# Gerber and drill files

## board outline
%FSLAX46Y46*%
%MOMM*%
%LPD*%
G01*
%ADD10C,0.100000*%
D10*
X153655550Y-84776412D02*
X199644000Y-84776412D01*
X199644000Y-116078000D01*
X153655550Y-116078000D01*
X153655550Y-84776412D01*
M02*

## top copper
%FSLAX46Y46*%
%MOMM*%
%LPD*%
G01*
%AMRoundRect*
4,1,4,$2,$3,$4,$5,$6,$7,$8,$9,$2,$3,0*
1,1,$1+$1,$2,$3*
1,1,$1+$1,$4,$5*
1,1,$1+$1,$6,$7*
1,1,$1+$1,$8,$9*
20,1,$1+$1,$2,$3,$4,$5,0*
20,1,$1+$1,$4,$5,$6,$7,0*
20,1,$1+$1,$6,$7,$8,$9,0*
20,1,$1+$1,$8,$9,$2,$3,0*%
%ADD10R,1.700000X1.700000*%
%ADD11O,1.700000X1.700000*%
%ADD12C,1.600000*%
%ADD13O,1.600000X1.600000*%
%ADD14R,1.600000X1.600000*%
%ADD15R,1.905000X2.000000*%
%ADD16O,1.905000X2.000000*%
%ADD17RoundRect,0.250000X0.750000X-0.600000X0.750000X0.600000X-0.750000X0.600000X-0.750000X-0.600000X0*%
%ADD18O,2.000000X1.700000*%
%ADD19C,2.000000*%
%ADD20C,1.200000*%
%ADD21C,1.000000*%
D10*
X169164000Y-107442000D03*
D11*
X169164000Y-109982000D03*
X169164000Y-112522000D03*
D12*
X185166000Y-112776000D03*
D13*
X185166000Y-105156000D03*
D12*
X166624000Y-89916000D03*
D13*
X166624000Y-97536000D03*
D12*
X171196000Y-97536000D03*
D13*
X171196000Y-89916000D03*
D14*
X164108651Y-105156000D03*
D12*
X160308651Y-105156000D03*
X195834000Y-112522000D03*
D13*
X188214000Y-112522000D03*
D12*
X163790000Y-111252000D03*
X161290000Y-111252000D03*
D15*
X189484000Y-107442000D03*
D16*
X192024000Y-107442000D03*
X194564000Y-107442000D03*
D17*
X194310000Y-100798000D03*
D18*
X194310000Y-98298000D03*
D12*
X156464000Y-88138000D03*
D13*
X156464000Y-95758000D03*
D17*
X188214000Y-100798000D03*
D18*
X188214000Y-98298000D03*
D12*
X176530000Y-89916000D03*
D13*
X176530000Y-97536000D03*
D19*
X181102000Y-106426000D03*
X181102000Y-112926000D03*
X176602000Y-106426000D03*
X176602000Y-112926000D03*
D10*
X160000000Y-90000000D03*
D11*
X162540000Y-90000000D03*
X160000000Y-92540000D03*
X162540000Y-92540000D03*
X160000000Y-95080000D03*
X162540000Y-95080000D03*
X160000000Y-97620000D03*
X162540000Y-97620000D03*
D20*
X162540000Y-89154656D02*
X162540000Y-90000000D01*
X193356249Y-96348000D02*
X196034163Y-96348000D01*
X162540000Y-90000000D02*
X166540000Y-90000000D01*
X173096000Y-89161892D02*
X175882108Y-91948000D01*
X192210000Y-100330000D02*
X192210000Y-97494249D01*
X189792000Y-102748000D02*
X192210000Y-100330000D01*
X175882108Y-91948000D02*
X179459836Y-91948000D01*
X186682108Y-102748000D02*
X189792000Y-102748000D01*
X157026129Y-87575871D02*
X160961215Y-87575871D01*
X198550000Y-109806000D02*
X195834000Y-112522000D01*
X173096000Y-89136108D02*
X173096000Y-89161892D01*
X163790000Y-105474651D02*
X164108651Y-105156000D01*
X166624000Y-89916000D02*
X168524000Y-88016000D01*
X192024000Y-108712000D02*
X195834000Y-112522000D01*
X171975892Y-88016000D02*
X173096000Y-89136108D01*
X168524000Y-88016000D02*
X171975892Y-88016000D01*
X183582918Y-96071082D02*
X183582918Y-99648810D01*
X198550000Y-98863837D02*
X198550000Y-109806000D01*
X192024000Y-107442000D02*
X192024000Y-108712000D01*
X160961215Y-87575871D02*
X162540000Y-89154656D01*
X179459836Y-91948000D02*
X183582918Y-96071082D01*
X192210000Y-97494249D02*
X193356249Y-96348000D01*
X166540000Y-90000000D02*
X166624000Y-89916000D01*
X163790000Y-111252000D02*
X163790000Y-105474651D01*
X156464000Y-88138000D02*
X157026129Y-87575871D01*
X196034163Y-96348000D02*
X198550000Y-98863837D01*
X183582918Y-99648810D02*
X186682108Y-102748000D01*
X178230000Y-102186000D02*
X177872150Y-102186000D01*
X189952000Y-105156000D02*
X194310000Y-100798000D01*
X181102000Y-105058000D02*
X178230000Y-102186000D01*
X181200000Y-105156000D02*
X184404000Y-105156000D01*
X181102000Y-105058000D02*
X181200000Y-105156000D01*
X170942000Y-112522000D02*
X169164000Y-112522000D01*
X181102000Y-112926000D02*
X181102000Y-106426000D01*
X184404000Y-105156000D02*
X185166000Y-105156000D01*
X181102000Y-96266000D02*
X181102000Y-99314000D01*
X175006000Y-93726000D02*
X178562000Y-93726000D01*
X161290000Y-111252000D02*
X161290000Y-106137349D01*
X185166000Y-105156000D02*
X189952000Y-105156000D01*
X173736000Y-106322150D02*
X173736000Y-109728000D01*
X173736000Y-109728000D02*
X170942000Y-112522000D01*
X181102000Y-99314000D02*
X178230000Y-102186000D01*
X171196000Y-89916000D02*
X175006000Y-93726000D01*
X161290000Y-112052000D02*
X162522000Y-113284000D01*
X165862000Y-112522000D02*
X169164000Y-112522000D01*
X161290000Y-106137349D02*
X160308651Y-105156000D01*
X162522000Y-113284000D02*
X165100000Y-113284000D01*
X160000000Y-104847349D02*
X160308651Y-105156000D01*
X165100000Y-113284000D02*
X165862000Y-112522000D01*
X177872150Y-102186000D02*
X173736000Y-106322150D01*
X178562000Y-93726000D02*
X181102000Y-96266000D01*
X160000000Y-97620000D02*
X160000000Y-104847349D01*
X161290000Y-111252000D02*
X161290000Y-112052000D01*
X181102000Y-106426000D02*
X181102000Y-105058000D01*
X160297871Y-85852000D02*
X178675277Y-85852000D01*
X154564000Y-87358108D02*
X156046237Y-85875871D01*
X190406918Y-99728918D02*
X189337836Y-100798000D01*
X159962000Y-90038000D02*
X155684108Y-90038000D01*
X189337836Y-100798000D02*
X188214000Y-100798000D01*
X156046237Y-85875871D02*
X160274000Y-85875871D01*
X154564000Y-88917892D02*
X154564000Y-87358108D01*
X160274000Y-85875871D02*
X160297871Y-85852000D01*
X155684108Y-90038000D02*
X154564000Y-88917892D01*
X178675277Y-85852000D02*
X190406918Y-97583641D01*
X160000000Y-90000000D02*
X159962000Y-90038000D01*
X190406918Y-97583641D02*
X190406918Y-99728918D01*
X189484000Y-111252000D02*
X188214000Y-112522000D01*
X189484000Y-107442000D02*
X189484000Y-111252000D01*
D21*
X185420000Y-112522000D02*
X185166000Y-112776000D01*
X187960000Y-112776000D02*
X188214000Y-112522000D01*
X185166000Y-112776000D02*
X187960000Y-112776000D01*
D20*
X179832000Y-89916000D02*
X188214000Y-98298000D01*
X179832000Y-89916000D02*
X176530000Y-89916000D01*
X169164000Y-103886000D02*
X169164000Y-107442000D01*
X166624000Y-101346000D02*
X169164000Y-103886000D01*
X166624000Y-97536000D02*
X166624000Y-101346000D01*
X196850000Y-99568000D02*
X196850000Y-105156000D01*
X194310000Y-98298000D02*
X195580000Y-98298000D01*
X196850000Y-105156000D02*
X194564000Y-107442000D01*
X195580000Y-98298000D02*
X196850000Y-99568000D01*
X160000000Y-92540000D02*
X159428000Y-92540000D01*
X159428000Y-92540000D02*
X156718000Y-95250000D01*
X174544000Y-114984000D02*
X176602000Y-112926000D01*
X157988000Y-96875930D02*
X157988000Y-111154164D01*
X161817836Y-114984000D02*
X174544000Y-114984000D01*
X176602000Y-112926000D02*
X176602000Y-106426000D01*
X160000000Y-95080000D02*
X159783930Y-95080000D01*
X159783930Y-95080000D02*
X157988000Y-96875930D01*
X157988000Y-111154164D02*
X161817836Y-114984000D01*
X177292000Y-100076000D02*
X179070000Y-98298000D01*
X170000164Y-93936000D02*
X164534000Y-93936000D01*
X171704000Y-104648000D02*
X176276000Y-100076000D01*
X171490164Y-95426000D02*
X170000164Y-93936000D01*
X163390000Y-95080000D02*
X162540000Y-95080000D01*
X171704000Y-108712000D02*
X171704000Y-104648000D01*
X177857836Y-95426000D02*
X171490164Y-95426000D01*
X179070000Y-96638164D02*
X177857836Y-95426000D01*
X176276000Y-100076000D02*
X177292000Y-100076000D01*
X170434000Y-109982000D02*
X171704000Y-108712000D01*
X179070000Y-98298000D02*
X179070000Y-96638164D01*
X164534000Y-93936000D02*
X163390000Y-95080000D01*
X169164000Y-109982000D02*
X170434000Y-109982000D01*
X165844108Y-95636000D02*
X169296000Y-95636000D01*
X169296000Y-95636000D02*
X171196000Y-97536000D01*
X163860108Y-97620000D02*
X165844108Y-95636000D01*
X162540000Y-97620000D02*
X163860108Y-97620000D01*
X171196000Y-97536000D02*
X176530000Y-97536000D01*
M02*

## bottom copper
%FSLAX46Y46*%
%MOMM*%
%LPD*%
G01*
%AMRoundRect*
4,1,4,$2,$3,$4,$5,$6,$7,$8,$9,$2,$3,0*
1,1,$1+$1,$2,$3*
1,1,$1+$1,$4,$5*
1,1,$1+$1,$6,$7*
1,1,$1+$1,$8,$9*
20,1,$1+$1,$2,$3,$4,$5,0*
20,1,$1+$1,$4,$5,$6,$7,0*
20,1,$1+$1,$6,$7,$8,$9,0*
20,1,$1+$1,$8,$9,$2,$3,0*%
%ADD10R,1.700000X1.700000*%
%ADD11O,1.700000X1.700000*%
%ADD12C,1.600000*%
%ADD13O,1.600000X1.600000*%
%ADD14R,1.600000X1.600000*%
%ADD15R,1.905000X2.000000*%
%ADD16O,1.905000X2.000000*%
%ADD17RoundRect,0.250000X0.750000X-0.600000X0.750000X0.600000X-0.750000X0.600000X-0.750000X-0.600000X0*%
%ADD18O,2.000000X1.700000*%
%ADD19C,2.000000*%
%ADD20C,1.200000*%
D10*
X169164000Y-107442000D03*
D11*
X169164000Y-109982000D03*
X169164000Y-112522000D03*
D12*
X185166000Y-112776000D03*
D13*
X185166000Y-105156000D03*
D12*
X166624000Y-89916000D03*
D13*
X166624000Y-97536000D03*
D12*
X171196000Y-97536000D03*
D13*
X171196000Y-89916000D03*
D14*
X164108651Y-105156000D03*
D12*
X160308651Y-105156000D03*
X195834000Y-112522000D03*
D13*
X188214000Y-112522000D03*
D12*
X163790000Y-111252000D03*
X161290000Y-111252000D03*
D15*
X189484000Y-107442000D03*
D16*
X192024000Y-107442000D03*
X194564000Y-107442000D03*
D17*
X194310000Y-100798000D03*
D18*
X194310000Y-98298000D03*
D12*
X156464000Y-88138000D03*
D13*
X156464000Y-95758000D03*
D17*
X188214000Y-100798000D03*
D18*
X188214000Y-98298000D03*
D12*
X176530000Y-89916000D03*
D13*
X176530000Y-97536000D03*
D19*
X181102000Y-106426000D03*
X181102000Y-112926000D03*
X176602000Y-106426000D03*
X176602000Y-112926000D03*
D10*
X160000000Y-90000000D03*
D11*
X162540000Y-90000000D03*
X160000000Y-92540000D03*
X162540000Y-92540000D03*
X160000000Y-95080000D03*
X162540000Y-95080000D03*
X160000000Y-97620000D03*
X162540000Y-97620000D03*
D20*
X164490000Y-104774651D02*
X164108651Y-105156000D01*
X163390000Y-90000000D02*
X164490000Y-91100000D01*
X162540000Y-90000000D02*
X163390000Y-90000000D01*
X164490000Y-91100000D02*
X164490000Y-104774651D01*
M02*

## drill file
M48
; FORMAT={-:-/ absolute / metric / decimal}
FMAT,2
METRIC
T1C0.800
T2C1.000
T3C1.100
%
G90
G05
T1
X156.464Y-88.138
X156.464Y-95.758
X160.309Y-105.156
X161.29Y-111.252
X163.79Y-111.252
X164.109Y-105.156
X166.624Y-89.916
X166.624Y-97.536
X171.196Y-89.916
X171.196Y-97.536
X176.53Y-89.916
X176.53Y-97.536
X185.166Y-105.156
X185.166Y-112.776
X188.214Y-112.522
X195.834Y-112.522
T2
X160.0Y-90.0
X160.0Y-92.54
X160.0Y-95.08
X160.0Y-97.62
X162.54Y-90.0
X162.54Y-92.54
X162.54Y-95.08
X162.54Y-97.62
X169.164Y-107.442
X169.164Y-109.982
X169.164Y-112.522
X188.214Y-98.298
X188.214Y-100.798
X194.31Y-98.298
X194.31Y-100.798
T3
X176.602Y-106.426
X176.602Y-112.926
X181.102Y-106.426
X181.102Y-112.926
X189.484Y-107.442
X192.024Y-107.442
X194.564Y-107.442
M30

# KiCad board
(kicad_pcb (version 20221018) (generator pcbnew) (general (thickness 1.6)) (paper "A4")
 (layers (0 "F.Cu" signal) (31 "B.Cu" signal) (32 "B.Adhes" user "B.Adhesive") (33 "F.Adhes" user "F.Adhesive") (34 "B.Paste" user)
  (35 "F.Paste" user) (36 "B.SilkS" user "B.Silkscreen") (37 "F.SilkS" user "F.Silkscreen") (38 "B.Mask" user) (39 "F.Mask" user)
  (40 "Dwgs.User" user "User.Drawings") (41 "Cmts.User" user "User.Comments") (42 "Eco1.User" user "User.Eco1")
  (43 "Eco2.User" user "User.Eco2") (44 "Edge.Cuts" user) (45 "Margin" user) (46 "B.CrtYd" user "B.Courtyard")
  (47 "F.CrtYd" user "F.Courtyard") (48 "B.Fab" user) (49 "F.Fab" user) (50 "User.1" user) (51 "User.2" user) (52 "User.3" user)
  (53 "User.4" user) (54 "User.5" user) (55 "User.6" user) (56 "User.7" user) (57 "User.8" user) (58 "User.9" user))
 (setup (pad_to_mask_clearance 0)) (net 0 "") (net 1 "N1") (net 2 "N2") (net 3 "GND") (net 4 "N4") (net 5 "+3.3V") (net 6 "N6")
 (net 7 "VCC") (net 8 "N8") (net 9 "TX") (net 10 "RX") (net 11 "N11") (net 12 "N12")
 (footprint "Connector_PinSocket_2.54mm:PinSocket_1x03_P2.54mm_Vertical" (layer "F.Cu") (at 169.164 107.442)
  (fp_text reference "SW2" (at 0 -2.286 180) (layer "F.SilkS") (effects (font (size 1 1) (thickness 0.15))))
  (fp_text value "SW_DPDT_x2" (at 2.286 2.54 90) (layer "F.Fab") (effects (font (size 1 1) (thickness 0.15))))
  (pad "1" thru_hole rect (at 0 0) (size 1.7 1.7) (drill 1) (layers "*.Cu" "*.Mask") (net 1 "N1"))
  (pad "2" thru_hole oval (at 0 2.54) (size 1.7 1.7) (drill 1) (layers "*.Cu" "*.Mask") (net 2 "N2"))
  (pad "3" thru_hole oval (at 0 5.08) (size 1.7 1.7) (drill 1) (layers "*.Cu" "*.Mask") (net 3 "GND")))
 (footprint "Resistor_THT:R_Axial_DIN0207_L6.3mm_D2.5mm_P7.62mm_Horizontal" (layer "F.Cu") (at 185.166 112.776 90)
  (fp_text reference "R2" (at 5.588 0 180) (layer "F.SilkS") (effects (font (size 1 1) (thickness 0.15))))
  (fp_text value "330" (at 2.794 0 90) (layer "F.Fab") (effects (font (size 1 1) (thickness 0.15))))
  (pad "1" thru_hole circle (at 0 0 90) (size 1.6 1.6) (drill 0.8) (layers "*.Cu" "*.Mask") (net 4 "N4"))
  (pad "2" thru_hole oval (at 7.62 0 90) (size 1.6 1.6) (drill 0.8) (layers "*.Cu" "*.Mask") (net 3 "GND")))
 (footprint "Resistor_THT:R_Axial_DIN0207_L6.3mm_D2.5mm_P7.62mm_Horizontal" (layer "F.Cu") (at 166.624 89.916 -90)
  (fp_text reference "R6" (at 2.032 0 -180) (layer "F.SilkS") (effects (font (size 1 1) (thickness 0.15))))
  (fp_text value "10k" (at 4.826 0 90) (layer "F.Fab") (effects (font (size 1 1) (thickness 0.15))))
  (pad "1" thru_hole circle (at 0 0 270) (size 1.6 1.6) (drill 0.8) (layers "*.Cu" "*.Mask") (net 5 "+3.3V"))
  (pad "2" thru_hole oval (at 7.62 0 270) (size 1.6 1.6) (drill 0.8) (layers "*.Cu" "*.Mask") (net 1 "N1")))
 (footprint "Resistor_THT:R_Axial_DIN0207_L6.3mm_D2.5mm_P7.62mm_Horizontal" (layer "F.Cu") (at 171.196 97.536 90)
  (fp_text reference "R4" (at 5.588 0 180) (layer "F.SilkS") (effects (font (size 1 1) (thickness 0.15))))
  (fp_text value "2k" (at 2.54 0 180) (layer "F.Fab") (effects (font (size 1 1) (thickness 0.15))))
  (pad "1" thru_hole circle (at 0 0 90) (size 1.6 1.6) (drill 0.8) (layers "*.Cu" "*.Mask") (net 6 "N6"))
  (pad "2" thru_hole oval (at 7.62 0 90) (size 1.6 1.6) (drill 0.8) (layers "*.Cu" "*.Mask") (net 3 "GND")))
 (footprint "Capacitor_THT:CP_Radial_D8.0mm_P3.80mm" (layer "F.Cu") (at 164.108651 105.156 180)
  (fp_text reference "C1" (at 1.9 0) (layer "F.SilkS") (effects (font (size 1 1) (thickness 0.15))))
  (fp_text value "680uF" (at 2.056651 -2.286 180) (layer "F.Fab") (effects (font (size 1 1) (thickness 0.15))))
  (pad "1" thru_hole rect (at 0 0 180) (size 1.6 1.6) (drill 0.8) (layers "*.Cu" "*.Mask") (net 5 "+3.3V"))
  (pad "2" thru_hole circle (at 3.8 0 180) (size 1.6 1.6) (drill 0.8) (layers "*.Cu" "*.Mask") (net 3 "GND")))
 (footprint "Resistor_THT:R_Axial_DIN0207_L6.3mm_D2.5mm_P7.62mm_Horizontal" (layer "F.Cu") (at 195.834 112.522 180)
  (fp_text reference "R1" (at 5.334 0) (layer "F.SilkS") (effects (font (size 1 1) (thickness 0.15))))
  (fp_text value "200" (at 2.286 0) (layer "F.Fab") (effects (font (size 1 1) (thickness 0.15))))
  (pad "1" thru_hole circle (at 0 0 180) (size 1.6 1.6) (drill 0.8) (layers "*.Cu" "*.Mask") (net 5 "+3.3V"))
  (pad "2" thru_hole oval (at 7.62 0 180) (size 1.6 1.6) (drill 0.8) (layers "*.Cu" "*.Mask") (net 4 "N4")))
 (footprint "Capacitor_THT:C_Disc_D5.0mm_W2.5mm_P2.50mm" (layer "F.Cu") (at 163.79 111.252 180)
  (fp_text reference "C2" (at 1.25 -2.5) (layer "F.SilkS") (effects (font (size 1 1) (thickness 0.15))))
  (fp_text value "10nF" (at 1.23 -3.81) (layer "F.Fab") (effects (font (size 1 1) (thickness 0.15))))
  (pad "1" thru_hole circle (at 0 0 180) (size 1.6 1.6) (drill 0.8) (layers "*.Cu" "*.Mask") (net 5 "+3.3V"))
  (pad "2" thru_hole circle (at 2.5 0 180) (size 1.6 1.6) (drill 0.8) (layers "*.Cu" "*.Mask") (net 3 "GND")))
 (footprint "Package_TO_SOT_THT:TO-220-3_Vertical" (layer "F.Cu") (at 189.484 107.442)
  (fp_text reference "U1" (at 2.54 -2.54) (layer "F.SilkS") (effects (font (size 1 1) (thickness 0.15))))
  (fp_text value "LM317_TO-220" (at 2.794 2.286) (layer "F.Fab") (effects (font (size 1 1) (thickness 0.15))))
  (pad "1" thru_hole rect (at 0 0) (size 1.905 2) (drill 1.1) (layers "*.Cu" "*.Mask") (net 4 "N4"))
  (pad "2" thru_hole oval (at 2.54 0) (size 1.905 2) (drill 1.1) (layers "*.Cu" "*.Mask") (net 5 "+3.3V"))
  (pad "3" thru_hole oval (at 5.08 0) (size 1.905 2) (drill 1.1) (layers "*.Cu" "*.Mask") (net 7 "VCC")))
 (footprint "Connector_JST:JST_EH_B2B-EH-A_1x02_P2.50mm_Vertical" (layer "F.Cu") (at 194.31 100.798 90)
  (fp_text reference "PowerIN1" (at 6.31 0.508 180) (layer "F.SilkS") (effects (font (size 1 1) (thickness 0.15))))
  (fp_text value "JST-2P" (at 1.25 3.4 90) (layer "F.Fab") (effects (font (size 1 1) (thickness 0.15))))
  (pad "1" thru_hole roundrect (at 0 0 90) (size 1.7 2) (drill 1) (layers "*.Cu" "*.Mask") (roundrect_rratio 0.147059) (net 3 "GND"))
  (pad "2" thru_hole oval (at 2.5 0 90) (size 1.7 2) (drill 1) (layers "*.Cu" "*.Mask") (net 7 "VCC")))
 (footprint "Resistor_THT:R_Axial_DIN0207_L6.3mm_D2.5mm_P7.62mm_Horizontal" (layer "F.Cu") (at 156.464 88.138 -90)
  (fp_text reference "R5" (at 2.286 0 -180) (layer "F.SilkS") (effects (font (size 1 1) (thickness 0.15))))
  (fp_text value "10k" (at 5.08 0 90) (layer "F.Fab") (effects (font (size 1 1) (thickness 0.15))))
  (pad "1" thru_hole circle (at 0 0 270) (size 1.6 1.6) (drill 0.8) (layers "*.Cu" "*.Mask") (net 5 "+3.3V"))
  (pad "2" thru_hole oval (at 7.62 0 270) (size 1.6 1.6) (drill 0.8) (layers "*.Cu" "*.Mask") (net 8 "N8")))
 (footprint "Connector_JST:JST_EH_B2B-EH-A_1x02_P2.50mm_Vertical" (layer "F.Cu") (at 188.214 100.798 90)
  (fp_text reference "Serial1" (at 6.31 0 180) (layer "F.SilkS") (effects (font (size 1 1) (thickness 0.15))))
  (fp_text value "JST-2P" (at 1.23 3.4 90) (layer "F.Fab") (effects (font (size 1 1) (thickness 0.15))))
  (pad "1" thru_hole roundrect (at 0 0 90) (size 1.7 2) (drill 1) (layers "*.Cu" "*.Mask") (roundrect_rratio 0.147059) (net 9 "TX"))
  (pad "2" thru_hole oval (at 2.5 0 90) (size 1.7 2) (drill 1) (layers "*.Cu" "*.Mask") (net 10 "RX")))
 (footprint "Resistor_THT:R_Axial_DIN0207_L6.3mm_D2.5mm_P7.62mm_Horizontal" (layer "F.Cu") (at 176.53 89.916 -90)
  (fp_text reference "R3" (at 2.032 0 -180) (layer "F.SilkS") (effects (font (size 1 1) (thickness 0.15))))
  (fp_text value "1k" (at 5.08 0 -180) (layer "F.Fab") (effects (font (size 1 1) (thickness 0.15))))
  (pad "1" thru_hole circle (at 0 0 270) (size 1.6 1.6) (drill 0.8) (layers "*.Cu" "*.Mask") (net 10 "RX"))
  (pad "2" thru_hole oval (at 7.62 0 270) (size 1.6 1.6) (drill 0.8) (layers "*.Cu" "*.Mask") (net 6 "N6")))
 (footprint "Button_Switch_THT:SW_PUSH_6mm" (layer "F.Cu") (at 181.102 106.426 -90)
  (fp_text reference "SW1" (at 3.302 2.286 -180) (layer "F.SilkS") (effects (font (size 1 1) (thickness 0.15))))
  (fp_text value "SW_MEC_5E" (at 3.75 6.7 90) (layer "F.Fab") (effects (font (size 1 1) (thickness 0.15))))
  (pad "1" thru_hole circle (at 0 0) (size 2 2) (drill 1.1) (layers "*.Cu" "*.Mask") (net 3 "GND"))
  (pad "1" thru_hole circle (at 6.5 0) (size 2 2) (drill 1.1) (layers "*.Cu" "*.Mask") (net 3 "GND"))
  (pad "2" thru_hole circle (at 0 4.5) (size 2 2) (drill 1.1) (layers "*.Cu" "*.Mask") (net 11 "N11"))
  (pad "2" thru_hole circle (at 6.5 4.5) (size 2 2) (drill 1.1) (layers "*.Cu" "*.Mask") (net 11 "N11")))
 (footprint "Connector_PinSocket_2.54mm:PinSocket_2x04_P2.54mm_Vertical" (layer "B.Cu") (at 160 90 180)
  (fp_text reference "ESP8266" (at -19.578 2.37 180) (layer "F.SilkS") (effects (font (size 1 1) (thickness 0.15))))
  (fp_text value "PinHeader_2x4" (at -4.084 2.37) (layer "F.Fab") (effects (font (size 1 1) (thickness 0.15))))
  (pad "1" thru_hole rect (at 0 0 180) (size 1.7 1.7) (drill 1) (layers "*.Cu" "*.Mask") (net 9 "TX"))
  (pad "2" thru_hole oval (at -2.54 0 180) (size 1.7 1.7) (drill 1) (layers "*.Cu" "*.Mask") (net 5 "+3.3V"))
  (pad "3" thru_hole oval (at 0 -2.54 180) (size 1.7 1.7) (drill 1) (layers "*.Cu" "*.Mask") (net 8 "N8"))
  (pad "4" thru_hole oval (at -2.54 -2.54 180) (size 1.7 1.7) (drill 1) (layers "*.Cu" "*.Mask") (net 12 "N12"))
  (pad "5" thru_hole oval (at 0 -5.08 180) (size 1.7 1.7) (drill 1) (layers "*.Cu" "*.Mask") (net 11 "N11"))
  (pad "6" thru_hole oval (at -2.54 -5.08 180) (size 1.7 1.7) (drill 1) (layers "*.Cu" "*.Mask") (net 2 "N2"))
  (pad "7" thru_hole oval (at 0 -7.62 180) (size 1.7 1.7) (drill 1) (layers "*.Cu" "*.Mask") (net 3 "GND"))
  (pad "8" thru_hole oval (at -2.54 -7.62 180) (size 1.7 1.7) (drill 1) (layers "*.Cu" "*.Mask") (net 6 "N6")))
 (gr_rect (start 153.65555 84.776412) (end 199.644 116.078) (stroke (width 0.1) (type default)) (fill none) (layer "Edge.Cuts"))
 (segment (start 162.54 89.154656) (end 162.54 90) (width 1.2) (layer "F.Cu") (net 5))
 (segment (start 193.356249 96.348) (end 196.034163 96.348) (width 1.2) (layer "F.Cu") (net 5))
 (segment (start 162.54 90) (end 166.54 90) (width 1.2) (layer "F.Cu") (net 5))
 (segment (start 173.096 89.161892) (end 175.882108 91.948) (width 1.2) (layer "F.Cu") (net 5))
 (segment (start 192.21 100.33) (end 192.21 97.494249) (width 1.2) (layer "F.Cu") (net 5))
 (segment (start 189.792 102.748) (end 192.21 100.33) (width 1.2) (layer "F.Cu") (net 5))
 (segment (start 175.882108 91.948) (end 179.459836 91.948) (width 1.2) (layer "F.Cu") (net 5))
 (segment (start 186.682108 102.748) (end 189.792 102.748) (width 1.2) (layer "F.Cu") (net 5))
 (segment (start 157.026129 87.575871) (end 160.961215 87.575871) (width 1.2) (layer "F.Cu") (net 5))
 (segment (start 198.55 109.806) (end 195.834 112.522) (width 1.2) (layer "F.Cu") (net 5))
 (segment (start 173.096 89.136108) (end 173.096 89.161892) (width 1.2) (layer "F.Cu") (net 5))
 (segment (start 163.79 105.474651) (end 164.108651 105.156) (width 1.2) (layer "F.Cu") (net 5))
 (segment (start 166.624 89.916) (end 168.524 88.016) (width 1.2) (layer "F.Cu") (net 5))
 (segment (start 192.024 108.712) (end 195.834 112.522) (width 1.2) (layer "F.Cu") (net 5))
 (segment (start 171.975892 88.016) (end 173.096 89.136108) (width 1.2) (layer "F.Cu") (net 5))
 (segment (start 168.524 88.016) (end 171.975892 88.016) (width 1.2) (layer "F.Cu") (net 5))
 (segment (start 183.582918 96.071082) (end 183.582918 99.64881) (width 1.2) (layer "F.Cu") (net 5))
 (segment (start 198.55 98.863837) (end 198.55 109.806) (width 1.2) (layer "F.Cu") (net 5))
 (segment (start 192.024 107.442) (end 192.024 108.712) (width 1.2) (layer "F.Cu") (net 5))
 (segment (start 160.961215 87.575871) (end 162.54 89.154656) (width 1.2) (layer "F.Cu") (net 5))
 (segment (start 179.459836 91.948) (end 183.582918 96.071082) (width 1.2) (layer "F.Cu") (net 5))
 (segment (start 192.21 97.494249) (end 193.356249 96.348) (width 1.2) (layer "F.Cu") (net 5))
 (segment (start 166.54 90) (end 166.624 89.916) (width 1.2) (layer "F.Cu") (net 5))
 (segment (start 163.79 111.252) (end 163.79 105.474651) (width 1.2) (layer "F.Cu") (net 5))
 (segment (start 156.464 88.138) (end 157.026129 87.575871) (width 1.2) (layer "F.Cu") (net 5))
 (segment (start 196.034163 96.348) (end 198.55 98.863837) (width 1.2) (layer "F.Cu") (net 5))
 (segment (start 183.582918 99.64881) (end 186.682108 102.748) (width 1.2) (layer "F.Cu") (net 5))
 (segment (start 164.49 104.774651) (end 164.108651 105.156) (width 1.2) (layer "B.Cu") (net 5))
 (segment (start 163.39 90) (end 164.49 91.1) (width 1.2) (layer "B.Cu") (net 5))
 (segment (start 162.54 90) (end 163.39 90) (width 1.2) (layer "B.Cu") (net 5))
 (segment (start 164.49 91.1) (end 164.49 104.774651) (width 1.2) (layer "B.Cu") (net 5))
 (segment (start 178.23 102.186) (end 177.87215 102.186) (width 1.2) (layer "F.Cu") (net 3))
 (segment (start 189.952 105.156) (end 194.31 100.798) (width 1.2) (layer "F.Cu") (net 3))
 (segment (start 181.102 105.058) (end 178.23 102.186) (width 1.2) (layer "F.Cu") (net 3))
 (segment (start 181.2 105.156) (end 184.404 105.156) (width 1.2) (layer "F.Cu") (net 3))
 (segment (start 181.102 105.058) (end 181.2 105.156) (width 1.2) (layer "F.Cu") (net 3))
 (segment (start 170.942 112.522) (end 169.164 112.522) (width 1.2) (layer "F.Cu") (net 3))
 (segment (start 181.102 112.926) (end 181.102 106.426) (width 1.2) (layer "F.Cu") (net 3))
 (segment (start 184.404 105.156) (end 185.166 105.156) (width 1.2) (layer "F.Cu") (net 3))
 (segment (start 181.102 96.266) (end 181.102 99.314) (width 1.2) (layer "F.Cu") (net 3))
 (segment (start 175.006 93.726) (end 178.562 93.726) (width 1.2) (layer "F.Cu") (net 3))
 (segment (start 161.29 111.252) (end 161.29 106.137349) (width 1.2) (layer "F.Cu") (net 3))
 (segment (start 185.166 105.156) (end 189.952 105.156) (width 1.2) (layer "F.Cu") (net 3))
 (segment (start 173.736 106.32215) (end 173.736 109.728) (width 1.2) (layer "F.Cu") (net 3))
 (segment (start 173.736 109.728) (end 170.942 112.522) (width 1.2) (layer "F.Cu") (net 3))
 (segment (start 181.102 99.314) (end 178.23 102.186) (width 1.2) (layer "F.Cu") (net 3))
 (segment (start 171.196 89.916) (end 175.006 93.726) (width 1.2) (layer "F.Cu") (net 3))
 (segment (start 161.29 112.052) (end 162.522 113.284) (width 1.2) (layer "F.Cu") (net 3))
 (segment (start 165.862 112.522) (end 169.164 112.522) (width 1.2) (layer "F.Cu") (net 3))
 (segment (start 161.29 106.137349) (end 160.308651 105.156) (width 1.2) (layer "F.Cu") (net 3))
 (segment (start 162.522 113.284) (end 165.1 113.284) (width 1.2) (layer "F.Cu") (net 3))
 (segment (start 160 104.847349) (end 160.308651 105.156) (width 1.2) (layer "F.Cu") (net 3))
 (segment (start 165.1 113.284) (end 165.862 112.522) (width 1.2) (layer "F.Cu") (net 3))
 (segment (start 177.87215 102.186) (end 173.736 106.32215) (width 1.2) (layer "F.Cu") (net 3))
 (segment (start 178.562 93.726) (end 181.102 96.266) (width 1.2) (layer "F.Cu") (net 3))
 (segment (start 160 97.62) (end 160 104.847349) (width 1.2) (layer "F.Cu") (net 3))
 (segment (start 161.29 111.252) (end 161.29 112.052) (width 1.2) (layer "F.Cu") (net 3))
 (segment (start 181.102 106.426) (end 181.102 105.058) (width 1.2) (layer "F.Cu") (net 3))
 (segment (start 160.297871 85.852) (end 178.675277 85.852) (width 1.2) (layer "F.Cu") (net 9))
 (segment (start 154.564 87.358108) (end 156.046237 85.875871) (width 1.2) (layer "F.Cu") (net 9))
 (segment (start 190.406918 99.728918) (end 189.337836 100.798) (width 1.2) (layer "F.Cu") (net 9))
 (segment (start 159.962 90.038) (end 155.684108 90.038) (width 1.2) (layer "F.Cu") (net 9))
 (segment (start 189.337836 100.798) (end 188.214 100.798) (width 1.2) (layer "F.Cu") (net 9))
 (segment (start 156.046237 85.875871) (end 160.274 85.875871) (width 1.2) (layer "F.Cu") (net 9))
 (segment (start 154.564 88.917892) (end 154.564 87.358108) (width 1.2) (layer "F.Cu") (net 9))
 (segment (start 160.274 85.875871) (end 160.297871 85.852) (width 1.2) (layer "F.Cu") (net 9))
 (segment (start 155.684108 90.038) (end 154.564 88.917892) (width 1.2) (layer "F.Cu") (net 9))
 (segment (start 178.675277 85.852) (end 190.406918 97.583641) (width 1.2) (layer "F.Cu") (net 9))
 (segment (start 160 90) (end 159.962 90.038) (width 1.2) (layer "F.Cu") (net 9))
 (segment (start 190.406918 97.583641) (end 190.406918 99.728918) (width 1.2) (layer "F.Cu") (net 9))
 (segment (start 189.484 111.252) (end 188.214 112.522) (width 1.2) (layer "F.Cu") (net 4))
 (segment (start 189.484 107.442) (end 189.484 111.252) (width 1.2) (layer "F.Cu") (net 4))
 (segment (start 185.42 112.522) (end 185.166 112.776) (width 1) (layer "F.Cu") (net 4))
 (segment (start 187.96 112.776) (end 188.214 112.522) (width 1) (layer "F.Cu") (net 4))
 (segment (start 185.166 112.776) (end 187.96 112.776) (width 1) (layer "F.Cu") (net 4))
 (segment (start 179.832 89.916) (end 188.214 98.298) (width 1.2) (layer "F.Cu") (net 10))
 (segment (start 179.832 89.916) (end 176.53 89.916) (width 1.2) (layer "F.Cu") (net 10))
 (segment (start 169.164 103.886) (end 169.164 107.442) (width 1.2) (layer "F.Cu") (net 1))
 (segment (start 166.624 101.346) (end 169.164 103.886) (width 1.2) (layer "F.Cu") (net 1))
 (segment (start 166.624 97.536) (end 166.624 101.346) (width 1.2) (layer "F.Cu") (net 1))
 (segment (start 196.85 99.568) (end 196.85 105.156) (width 1.2) (layer "F.Cu") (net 7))
 (segment (start 194.31 98.298) (end 195.58 98.298) (width 1.2) (layer "F.Cu") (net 7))
 (segment (start 196.85 105.156) (end 194.564 107.442) (width 1.2) (layer "F.Cu") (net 7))
 (segment (start 195.58 98.298) (end 196.85 99.568) (width 1.2) (layer "F.Cu") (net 7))
 (segment (start 160 92.54) (end 159.428 92.54) (width 1.2) (layer "F.Cu") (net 8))
 (segment (start 159.428 92.54) (end 156.718 95.25) (width 1.2) (layer "F.Cu") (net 8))
 (segment (start 174.544 114.984) (end 176.602 112.926) (width 1.2) (layer "F.Cu") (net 11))
 (segment (start 157.988 96.87593) (end 157.988 111.154164) (width 1.2) (layer "F.Cu") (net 11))
 (segment (start 161.817836 114.984) (end 174.544 114.984) (width 1.2) (layer "F.Cu") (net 11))
 (segment (start 176.602 112.926) (end 176.602 106.426) (width 1.2) (layer "F.Cu") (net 11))
 (segment (start 160 95.08) (end 159.78393 95.08) (width 1.2) (layer "F.Cu") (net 11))
 (segment (start 159.78393 95.08) (end 157.988 96.87593) (width 1.2) (layer "F.Cu") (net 11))
 (segment (start 157.988 111.154164) (end 161.817836 114.984) (width 1.2) (layer "F.Cu") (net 11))
 (segment (start 177.292 100.076) (end 179.07 98.298) (width 1.2) (layer "F.Cu") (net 2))
 (segment (start 170.000164 93.936) (end 164.534 93.936) (width 1.2) (layer "F.Cu") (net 2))
 (segment (start 171.704 104.648) (end 176.276 100.076) (width 1.2) (layer "F.Cu") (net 2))
 (segment (start 171.490164 95.426) (end 170.000164 93.936) (width 1.2) (layer "F.Cu") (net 2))
 (segment (start 163.39 95.08) (end 162.54 95.08) (width 1.2) (layer "F.Cu") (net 2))
 (segment (start 171.704 108.712) (end 171.704 104.648) (width 1.2) (layer "F.Cu") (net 2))
 (segment (start 177.857836 95.426) (end 171.490164 95.426) (width 1.2) (layer "F.Cu") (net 2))
 (segment (start 179.07 96.638164) (end 177.857836 95.426) (width 1.2) (layer "F.Cu") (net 2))
 (segment (start 176.276 100.076) (end 177.292 100.076) (width 1.2) (layer "F.Cu") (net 2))
 (segment (start 170.434 109.982) (end 171.704 108.712) (width 1.2) (layer "F.Cu") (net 2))
 (segment (start 179.07 98.298) (end 179.07 96.638164) (width 1.2) (layer "F.Cu") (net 2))
 (segment (start 164.534 93.936) (end 163.39 95.08) (width 1.2) (layer "F.Cu") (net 2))
 (segment (start 169.164 109.982) (end 170.434 109.982) (width 1.2) (layer "F.Cu") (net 2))
 (segment (start 165.844108 95.636) (end 169.296 95.636) (width 1.2) (layer "F.Cu") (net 6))
 (segment (start 169.296 95.636) (end 171.196 97.536) (width 1.2) (layer "F.Cu") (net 6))
 (segment (start 163.860108 97.62) (end 165.844108 95.636) (width 1.2) (layer "F.Cu") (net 6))
 (segment (start 162.54 97.62) (end 163.860108 97.62) (width 1.2) (layer "F.Cu") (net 6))
 (segment (start 171.196 97.536) (end 176.53 97.536) (width 1.2) (layer "F.Cu") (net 6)))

